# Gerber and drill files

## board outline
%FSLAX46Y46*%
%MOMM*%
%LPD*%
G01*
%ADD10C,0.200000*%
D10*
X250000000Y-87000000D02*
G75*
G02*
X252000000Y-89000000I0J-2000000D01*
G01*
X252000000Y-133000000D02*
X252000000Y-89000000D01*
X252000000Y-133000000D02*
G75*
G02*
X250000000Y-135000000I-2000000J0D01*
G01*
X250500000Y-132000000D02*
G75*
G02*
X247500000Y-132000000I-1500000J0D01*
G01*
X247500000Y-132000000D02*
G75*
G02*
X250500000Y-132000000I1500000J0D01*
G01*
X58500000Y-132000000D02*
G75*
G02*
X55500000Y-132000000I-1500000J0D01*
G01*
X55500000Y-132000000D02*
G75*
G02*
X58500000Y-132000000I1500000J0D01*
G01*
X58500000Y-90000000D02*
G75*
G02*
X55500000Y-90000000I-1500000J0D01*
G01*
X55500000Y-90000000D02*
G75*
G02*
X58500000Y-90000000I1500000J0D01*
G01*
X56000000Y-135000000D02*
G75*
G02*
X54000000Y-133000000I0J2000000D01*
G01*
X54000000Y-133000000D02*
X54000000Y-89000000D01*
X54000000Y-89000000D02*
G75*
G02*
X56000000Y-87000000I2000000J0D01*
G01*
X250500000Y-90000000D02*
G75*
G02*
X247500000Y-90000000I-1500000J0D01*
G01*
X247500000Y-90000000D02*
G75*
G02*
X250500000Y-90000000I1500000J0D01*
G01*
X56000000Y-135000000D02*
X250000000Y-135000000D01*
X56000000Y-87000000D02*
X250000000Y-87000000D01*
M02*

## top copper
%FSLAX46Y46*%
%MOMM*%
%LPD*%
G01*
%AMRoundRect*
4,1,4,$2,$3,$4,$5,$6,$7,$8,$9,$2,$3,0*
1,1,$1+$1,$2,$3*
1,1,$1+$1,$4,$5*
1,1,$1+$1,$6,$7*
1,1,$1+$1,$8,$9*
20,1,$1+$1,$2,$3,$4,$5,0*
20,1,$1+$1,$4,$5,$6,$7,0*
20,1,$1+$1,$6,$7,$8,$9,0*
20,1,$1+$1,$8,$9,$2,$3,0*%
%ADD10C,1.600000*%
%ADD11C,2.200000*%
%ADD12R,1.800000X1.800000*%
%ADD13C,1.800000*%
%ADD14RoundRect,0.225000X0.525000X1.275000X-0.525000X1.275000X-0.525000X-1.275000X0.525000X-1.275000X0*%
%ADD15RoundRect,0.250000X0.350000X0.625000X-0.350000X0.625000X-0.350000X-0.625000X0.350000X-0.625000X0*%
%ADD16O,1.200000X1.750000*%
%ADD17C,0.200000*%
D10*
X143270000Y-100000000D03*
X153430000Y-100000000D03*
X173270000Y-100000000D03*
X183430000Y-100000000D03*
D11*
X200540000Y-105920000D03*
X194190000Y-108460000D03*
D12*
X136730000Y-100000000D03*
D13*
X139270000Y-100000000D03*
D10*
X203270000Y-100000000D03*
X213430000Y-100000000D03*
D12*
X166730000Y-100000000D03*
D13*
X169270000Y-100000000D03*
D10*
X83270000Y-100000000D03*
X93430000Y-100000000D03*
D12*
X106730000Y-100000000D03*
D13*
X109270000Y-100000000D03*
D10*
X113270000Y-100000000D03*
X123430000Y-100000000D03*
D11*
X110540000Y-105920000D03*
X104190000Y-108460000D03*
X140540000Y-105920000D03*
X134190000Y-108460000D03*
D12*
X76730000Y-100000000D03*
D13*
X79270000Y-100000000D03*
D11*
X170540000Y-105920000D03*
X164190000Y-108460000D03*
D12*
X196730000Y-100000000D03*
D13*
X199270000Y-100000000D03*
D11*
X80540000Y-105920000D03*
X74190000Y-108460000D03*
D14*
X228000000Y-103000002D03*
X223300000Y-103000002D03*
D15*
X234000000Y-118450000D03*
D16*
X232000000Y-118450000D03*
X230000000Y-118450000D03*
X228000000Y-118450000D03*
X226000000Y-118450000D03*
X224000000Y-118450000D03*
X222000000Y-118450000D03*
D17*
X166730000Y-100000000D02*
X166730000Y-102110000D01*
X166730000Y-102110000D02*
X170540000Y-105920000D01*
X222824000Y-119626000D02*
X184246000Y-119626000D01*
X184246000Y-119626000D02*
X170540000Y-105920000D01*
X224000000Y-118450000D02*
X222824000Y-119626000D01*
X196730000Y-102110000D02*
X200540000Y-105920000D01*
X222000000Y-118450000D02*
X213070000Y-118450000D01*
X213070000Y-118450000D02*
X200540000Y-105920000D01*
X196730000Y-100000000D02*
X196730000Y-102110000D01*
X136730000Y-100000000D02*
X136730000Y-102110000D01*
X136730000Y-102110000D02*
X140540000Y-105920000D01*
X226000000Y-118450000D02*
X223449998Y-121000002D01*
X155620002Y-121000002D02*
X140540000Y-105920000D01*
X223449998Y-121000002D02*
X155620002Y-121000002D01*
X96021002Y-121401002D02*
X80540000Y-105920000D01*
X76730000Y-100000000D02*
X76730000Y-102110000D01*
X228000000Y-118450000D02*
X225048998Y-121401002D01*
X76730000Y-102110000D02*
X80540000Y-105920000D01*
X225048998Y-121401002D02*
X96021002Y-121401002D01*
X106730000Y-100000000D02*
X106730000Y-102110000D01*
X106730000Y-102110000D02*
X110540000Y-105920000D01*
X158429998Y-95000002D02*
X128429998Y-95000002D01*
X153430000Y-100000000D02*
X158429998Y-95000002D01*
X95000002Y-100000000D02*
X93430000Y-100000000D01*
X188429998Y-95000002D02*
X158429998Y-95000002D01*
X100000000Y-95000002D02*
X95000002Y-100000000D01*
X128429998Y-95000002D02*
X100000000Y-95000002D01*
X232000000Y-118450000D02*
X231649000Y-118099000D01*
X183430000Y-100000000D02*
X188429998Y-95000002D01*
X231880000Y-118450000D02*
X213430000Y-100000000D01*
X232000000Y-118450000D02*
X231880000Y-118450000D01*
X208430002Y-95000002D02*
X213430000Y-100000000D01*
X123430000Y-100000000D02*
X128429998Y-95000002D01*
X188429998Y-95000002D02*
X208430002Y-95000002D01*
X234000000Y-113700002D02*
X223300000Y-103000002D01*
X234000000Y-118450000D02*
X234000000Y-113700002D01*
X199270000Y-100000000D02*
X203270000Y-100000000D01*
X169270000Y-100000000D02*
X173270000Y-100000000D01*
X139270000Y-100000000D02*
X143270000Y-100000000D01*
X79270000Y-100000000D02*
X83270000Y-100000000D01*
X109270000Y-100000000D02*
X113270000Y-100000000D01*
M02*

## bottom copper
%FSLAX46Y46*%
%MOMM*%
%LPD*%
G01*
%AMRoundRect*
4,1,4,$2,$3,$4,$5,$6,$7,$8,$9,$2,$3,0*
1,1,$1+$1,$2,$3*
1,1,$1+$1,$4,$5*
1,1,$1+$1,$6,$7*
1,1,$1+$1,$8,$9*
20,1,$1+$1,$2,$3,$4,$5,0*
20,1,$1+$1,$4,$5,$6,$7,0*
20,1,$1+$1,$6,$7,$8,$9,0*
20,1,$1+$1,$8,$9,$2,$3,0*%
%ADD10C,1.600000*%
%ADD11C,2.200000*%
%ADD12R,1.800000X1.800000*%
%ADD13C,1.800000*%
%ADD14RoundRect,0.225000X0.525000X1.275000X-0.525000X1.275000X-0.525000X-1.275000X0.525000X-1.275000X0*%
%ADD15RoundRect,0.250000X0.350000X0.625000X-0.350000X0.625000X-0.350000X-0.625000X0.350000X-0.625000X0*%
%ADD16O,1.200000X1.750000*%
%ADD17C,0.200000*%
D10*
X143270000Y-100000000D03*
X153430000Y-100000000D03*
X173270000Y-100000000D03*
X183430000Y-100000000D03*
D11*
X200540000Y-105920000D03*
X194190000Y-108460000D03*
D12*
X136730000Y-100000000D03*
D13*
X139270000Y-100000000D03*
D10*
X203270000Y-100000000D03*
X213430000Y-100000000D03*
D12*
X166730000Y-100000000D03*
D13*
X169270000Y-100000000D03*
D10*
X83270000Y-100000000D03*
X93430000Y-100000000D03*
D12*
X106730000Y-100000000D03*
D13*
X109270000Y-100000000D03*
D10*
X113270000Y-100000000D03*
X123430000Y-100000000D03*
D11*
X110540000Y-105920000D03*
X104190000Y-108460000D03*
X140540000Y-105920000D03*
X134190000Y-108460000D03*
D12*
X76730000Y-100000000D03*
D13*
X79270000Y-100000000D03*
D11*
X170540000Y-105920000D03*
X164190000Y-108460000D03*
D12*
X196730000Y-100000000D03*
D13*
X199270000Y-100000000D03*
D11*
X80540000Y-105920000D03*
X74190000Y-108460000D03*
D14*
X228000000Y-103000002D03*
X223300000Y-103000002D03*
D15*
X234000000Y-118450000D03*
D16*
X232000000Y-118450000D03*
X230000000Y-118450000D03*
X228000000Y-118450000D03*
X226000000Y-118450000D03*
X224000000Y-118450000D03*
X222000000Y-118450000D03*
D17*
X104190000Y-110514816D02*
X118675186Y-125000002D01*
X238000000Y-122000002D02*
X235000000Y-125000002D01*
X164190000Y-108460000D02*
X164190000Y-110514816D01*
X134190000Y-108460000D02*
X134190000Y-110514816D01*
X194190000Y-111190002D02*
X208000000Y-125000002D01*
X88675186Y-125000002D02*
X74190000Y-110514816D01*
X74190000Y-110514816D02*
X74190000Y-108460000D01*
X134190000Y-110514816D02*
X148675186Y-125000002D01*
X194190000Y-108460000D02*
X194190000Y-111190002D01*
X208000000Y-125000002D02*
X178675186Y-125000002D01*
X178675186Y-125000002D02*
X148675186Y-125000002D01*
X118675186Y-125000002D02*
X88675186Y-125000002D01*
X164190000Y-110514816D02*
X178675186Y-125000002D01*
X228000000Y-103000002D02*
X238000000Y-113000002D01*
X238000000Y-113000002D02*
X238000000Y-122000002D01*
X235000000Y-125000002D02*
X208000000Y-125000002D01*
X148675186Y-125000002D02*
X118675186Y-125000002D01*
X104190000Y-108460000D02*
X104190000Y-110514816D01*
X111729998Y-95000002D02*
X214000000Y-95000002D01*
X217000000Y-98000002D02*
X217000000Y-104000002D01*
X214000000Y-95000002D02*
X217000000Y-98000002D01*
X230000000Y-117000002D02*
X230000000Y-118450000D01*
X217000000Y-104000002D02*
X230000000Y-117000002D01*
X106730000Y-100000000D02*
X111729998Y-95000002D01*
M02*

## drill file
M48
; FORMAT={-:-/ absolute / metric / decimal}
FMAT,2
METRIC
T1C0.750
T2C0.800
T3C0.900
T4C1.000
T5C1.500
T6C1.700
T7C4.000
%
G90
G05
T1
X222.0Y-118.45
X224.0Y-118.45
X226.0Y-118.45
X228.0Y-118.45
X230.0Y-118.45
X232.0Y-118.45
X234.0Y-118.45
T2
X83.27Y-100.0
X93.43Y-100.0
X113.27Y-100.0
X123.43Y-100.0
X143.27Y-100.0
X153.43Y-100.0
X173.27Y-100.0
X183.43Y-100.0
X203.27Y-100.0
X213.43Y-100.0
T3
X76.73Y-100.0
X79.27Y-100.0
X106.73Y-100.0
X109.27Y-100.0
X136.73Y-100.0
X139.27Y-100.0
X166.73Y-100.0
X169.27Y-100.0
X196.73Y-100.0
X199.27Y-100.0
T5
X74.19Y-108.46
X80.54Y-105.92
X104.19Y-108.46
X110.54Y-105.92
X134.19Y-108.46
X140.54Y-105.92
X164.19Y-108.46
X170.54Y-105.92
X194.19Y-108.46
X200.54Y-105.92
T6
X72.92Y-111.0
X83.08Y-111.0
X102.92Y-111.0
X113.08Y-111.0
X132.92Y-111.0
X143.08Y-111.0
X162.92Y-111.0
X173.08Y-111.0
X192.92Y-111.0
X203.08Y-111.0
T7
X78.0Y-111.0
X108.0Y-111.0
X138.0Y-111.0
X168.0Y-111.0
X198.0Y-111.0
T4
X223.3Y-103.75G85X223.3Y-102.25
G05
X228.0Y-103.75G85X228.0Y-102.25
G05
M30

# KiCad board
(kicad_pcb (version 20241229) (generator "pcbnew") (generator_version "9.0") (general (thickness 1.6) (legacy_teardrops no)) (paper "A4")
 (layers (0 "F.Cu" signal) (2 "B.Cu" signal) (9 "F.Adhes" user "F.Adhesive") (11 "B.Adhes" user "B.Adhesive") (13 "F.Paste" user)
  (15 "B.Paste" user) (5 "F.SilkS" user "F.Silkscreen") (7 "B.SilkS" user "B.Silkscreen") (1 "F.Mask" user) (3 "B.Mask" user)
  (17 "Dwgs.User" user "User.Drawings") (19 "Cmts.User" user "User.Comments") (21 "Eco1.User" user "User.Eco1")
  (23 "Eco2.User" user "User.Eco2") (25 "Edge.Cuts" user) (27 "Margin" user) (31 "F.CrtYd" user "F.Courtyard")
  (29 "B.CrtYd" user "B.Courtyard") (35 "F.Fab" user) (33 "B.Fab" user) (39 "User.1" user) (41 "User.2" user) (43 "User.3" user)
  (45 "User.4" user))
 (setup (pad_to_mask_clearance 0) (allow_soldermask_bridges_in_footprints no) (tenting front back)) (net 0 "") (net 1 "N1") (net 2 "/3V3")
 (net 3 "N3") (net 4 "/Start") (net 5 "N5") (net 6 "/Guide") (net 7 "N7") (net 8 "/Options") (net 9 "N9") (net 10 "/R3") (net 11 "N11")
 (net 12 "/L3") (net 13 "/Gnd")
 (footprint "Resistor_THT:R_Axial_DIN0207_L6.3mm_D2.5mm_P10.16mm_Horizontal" (layer "F.Cu") (at 143.27 100)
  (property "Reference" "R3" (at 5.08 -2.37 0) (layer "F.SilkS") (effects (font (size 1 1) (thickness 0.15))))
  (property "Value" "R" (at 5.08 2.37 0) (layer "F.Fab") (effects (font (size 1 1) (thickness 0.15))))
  (pad "1" thru_hole circle (at 0 0) (size 1.6 1.6) (drill 0.8) (layers "*.Cu" "*.Mask") (remove_unused_layers no) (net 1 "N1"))
  (pad "2" thru_hole circle (at 10.16 0) (size 1.6 1.6) (drill 0.8) (layers "*.Cu" "*.Mask") (remove_unused_layers no) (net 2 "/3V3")))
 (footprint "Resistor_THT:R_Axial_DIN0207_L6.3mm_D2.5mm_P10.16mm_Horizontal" (layer "F.Cu") (at 173.27 100)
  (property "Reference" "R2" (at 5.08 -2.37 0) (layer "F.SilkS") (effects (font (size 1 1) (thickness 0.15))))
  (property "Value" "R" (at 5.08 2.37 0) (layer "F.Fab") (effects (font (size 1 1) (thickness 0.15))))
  (pad "1" thru_hole circle (at 0 0) (size 1.6 1.6) (drill 0.8) (layers "*.Cu" "*.Mask") (remove_unused_layers no) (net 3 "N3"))
  (pad "2" thru_hole circle (at 10.16 0) (size 1.6 1.6) (drill 0.8) (layers "*.Cu" "*.Mask") (remove_unused_layers no) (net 2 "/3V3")))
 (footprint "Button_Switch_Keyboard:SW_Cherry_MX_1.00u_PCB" (layer "F.Cu") (at 200.54 105.92)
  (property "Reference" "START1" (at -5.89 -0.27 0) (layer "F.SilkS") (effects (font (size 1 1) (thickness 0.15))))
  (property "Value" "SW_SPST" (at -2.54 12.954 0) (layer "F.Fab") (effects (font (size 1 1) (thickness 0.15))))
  (pad "" np_thru_hole circle (at -7.62 5.08) (size 1.7 1.7) (drill 1.7) (layers "*.Cu" "*.Mask"))
  (pad "" np_thru_hole circle (at -2.54 5.08) (size 4 4) (drill 4) (layers "*.Cu" "*.Mask"))
  (pad "" np_thru_hole circle (at 2.54 5.08) (size 1.7 1.7) (drill 1.7) (layers "*.Cu" "*.Mask"))
  (pad "1" thru_hole circle (at 0 0) (size 2.2 2.2) (drill 1.5) (layers "*.Cu" "*.Mask") (remove_unused_layers no) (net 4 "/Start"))
  (pad "2" thru_hole circle (at -6.35 2.54) (size 2.2 2.2) (drill 1.5) (layers "*.Cu" "*.Mask") (remove_unused_layers no) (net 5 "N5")))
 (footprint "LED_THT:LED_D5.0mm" (layer "F.Cu") (at 136.73 100)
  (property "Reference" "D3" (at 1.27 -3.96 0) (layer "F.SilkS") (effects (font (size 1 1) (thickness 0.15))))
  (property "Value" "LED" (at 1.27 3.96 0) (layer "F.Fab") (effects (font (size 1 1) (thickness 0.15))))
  (pad "1" thru_hole rect (at 0 0) (size 1.8 1.8) (drill 0.9) (layers "*.Cu" "*.Mask") (remove_unused_layers no) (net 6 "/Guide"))
  (pad "2" thru_hole circle (at 2.54 0) (size 1.8 1.8) (drill 0.9) (layers "*.Cu" "*.Mask") (remove_unused_layers no) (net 1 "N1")))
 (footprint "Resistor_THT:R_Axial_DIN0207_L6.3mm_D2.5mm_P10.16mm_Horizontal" (layer "F.Cu") (at 203.27 100)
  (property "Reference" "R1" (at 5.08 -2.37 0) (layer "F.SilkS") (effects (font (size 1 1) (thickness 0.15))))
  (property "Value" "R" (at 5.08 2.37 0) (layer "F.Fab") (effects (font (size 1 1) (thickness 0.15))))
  (pad "1" thru_hole circle (at 0 0) (size 1.6 1.6) (drill 0.8) (layers "*.Cu" "*.Mask") (remove_unused_layers no) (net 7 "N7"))
  (pad "2" thru_hole circle (at 10.16 0) (size 1.6 1.6) (drill 0.8) (layers "*.Cu" "*.Mask") (remove_unused_layers no) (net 2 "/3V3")))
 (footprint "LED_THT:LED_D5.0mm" (layer "F.Cu") (at 166.73 100)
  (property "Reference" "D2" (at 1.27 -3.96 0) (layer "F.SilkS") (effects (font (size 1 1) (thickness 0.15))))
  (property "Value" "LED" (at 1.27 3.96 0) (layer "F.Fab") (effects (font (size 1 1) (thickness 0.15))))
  (pad "1" thru_hole rect (at 0 0) (size 1.8 1.8) (drill 0.9) (layers "*.Cu" "*.Mask") (remove_unused_layers no) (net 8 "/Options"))
  (pad "2" thru_hole circle (at 2.54 0) (size 1.8 1.8) (drill 0.9) (layers "*.Cu" "*.Mask") (remove_unused_layers no) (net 3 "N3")))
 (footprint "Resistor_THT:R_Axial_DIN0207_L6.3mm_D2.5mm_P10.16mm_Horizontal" (layer "F.Cu") (at 83.27 100)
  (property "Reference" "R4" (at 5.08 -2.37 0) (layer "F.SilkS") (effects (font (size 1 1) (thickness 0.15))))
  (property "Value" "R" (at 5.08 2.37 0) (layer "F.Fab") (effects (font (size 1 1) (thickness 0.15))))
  (pad "1" thru_hole circle (at 0 0) (size 1.6 1.6) (drill 0.8) (layers "*.Cu" "*.Mask") (remove_unused_layers no) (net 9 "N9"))
  (pad "2" thru_hole circle (at 10.16 0) (size 1.6 1.6) (drill 0.8) (layers "*.Cu" "*.Mask") (remove_unused_layers no) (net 2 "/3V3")))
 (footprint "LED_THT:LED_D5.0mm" (layer "F.Cu") (at 106.73 100)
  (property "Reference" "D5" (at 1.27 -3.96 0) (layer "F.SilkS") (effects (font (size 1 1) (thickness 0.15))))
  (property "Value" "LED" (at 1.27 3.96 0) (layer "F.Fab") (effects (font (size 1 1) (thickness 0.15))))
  (pad "1" thru_hole rect (at 0 0) (size 1.8 1.8) (drill 0.9) (layers "*.Cu" "*.Mask") (remove_unused_layers no) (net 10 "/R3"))
  (pad "2" thru_hole circle (at 2.54 0) (size 1.8 1.8) (drill 0.9) (layers "*.Cu" "*.Mask") (remove_unused_layers no) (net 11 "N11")))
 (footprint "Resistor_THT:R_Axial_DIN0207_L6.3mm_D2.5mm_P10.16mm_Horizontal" (layer "F.Cu") (at 113.27 100)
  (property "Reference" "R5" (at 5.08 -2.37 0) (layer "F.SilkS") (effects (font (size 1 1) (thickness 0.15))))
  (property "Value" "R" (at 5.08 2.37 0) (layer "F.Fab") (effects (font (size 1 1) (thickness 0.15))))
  (pad "1" thru_hole circle (at 0 0) (size 1.6 1.6) (drill 0.8) (layers "*.Cu" "*.Mask") (remove_unused_layers no) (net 11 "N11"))
  (pad "2" thru_hole circle (at 10.16 0) (size 1.6 1.6) (drill 0.8) (layers "*.Cu" "*.Mask") (remove_unused_layers no) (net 2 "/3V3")))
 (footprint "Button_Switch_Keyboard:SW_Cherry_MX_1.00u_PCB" (layer "F.Cu") (at 110.54 105.92)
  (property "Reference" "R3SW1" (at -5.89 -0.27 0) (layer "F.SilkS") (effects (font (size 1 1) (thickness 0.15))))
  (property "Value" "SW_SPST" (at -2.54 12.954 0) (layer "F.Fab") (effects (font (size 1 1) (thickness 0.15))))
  (pad "" np_thru_hole circle (at -7.62 5.08) (size 1.7 1.7) (drill 1.7) (layers "*.Cu" "*.Mask"))
  (pad "" np_thru_hole circle (at -2.54 5.08) (size 4 4) (drill 4) (layers "*.Cu" "*.Mask"))
  (pad "" np_thru_hole circle (at 2.54 5.08) (size 1.7 1.7) (drill 1.7) (layers "*.Cu" "*.Mask"))
  (pad "1" thru_hole circle (at 0 0) (size 2.2 2.2) (drill 1.5) (layers "*.Cu" "*.Mask") (remove_unused_layers no) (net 10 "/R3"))
  (pad "2" thru_hole circle (at -6.35 2.54) (size 2.2 2.2) (drill 1.5) (layers "*.Cu" "*.Mask") (remove_unused_layers no) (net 5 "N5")))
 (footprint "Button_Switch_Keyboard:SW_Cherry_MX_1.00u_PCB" (layer "F.Cu") (at 140.54 105.92)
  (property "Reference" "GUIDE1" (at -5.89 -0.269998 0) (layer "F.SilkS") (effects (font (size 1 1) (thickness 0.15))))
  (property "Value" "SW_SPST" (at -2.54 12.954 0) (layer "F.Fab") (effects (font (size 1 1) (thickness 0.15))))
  (pad "" np_thru_hole circle (at -7.62 5.08) (size 1.7 1.7) (drill 1.7) (layers "*.Cu" "*.Mask"))
  (pad "" np_thru_hole circle (at -2.54 5.08) (size 4 4) (drill 4) (layers "*.Cu" "*.Mask"))
  (pad "" np_thru_hole circle (at 2.54 5.08) (size 1.7 1.7) (drill 1.7) (layers "*.Cu" "*.Mask"))
  (pad "1" thru_hole circle (at 0 0) (size 2.2 2.2) (drill 1.5) (layers "*.Cu" "*.Mask") (remove_unused_layers no) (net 6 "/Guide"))
  (pad "2" thru_hole circle (at -6.35 2.54) (size 2.2 2.2) (drill 1.5) (layers "*.Cu" "*.Mask") (remove_unused_layers no) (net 5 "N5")))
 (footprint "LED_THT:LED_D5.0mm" (layer "F.Cu") (at 76.73 100)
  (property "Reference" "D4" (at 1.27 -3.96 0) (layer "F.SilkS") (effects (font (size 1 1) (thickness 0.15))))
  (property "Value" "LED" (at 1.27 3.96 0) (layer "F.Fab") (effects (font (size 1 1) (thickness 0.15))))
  (pad "1" thru_hole rect (at 0 0) (size 1.8 1.8) (drill 0.9) (layers "*.Cu" "*.Mask") (remove_unused_layers no) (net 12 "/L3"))
  (pad "2" thru_hole circle (at 2.54 0) (size 1.8 1.8) (drill 0.9) (layers "*.Cu" "*.Mask") (remove_unused_layers no) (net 9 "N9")))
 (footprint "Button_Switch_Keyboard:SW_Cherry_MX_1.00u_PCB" (layer "F.Cu") (at 170.54 105.92)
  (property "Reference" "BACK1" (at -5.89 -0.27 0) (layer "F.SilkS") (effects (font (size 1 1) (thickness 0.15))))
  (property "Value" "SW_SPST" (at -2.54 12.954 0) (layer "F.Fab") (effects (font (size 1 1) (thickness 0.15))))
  (pad "" np_thru_hole circle (at -7.62 5.08) (size 1.7 1.7) (drill 1.7) (layers "*.Cu" "*.Mask"))
  (pad "" np_thru_hole circle (at -2.54 5.08) (size 4 4) (drill 4) (layers "*.Cu" "*.Mask"))
  (pad "" np_thru_hole circle (at 2.54 5.08) (size 1.7 1.7) (drill 1.7) (layers "*.Cu" "*.Mask"))
  (pad "1" thru_hole circle (at 0 0) (size 2.2 2.2) (drill 1.5) (layers "*.Cu" "*.Mask") (remove_unused_layers no) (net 8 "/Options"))
  (pad "2" thru_hole circle (at -6.35 2.54) (size 2.2 2.2) (drill 1.5) (layers "*.Cu" "*.Mask") (remove_unused_layers no) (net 5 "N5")))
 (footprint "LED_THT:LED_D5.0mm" (layer "F.Cu") (at 196.73 100)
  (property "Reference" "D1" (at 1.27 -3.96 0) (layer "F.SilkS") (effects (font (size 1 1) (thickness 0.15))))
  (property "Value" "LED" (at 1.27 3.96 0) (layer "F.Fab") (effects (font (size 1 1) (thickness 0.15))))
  (pad "1" thru_hole rect (at 0 0) (size 1.8 1.8) (drill 0.9) (layers "*.Cu" "*.Mask") (remove_unused_layers no) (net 4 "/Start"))
  (pad "2" thru_hole circle (at 2.54 0) (size 1.8 1.8) (drill 0.9) (layers "*.Cu" "*.Mask") (remove_unused_layers no) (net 7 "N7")))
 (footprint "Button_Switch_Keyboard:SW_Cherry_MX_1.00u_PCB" (layer "F.Cu") (at 80.54 105.92)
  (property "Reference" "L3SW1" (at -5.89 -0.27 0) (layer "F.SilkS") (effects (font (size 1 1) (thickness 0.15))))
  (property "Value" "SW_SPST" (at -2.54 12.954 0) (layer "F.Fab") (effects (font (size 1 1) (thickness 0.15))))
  (pad "" np_thru_hole circle (at -7.62 5.08) (size 1.7 1.7) (drill 1.7) (layers "*.Cu" "*.Mask"))
  (pad "" np_thru_hole circle (at -2.54 5.08) (size 4 4) (drill 4) (layers "*.Cu" "*.Mask"))
  (pad "" np_thru_hole circle (at 2.54 5.08) (size 1.7 1.7) (drill 1.7) (layers "*.Cu" "*.Mask"))
  (pad "1" thru_hole circle (at 0 0) (size 2.2 2.2) (drill 1.5) (layers "*.Cu" "*.Mask") (remove_unused_layers no) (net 12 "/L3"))
  (pad "2" thru_hole circle (at -6.35 2.54) (size 2.2 2.2) (drill 1.5) (layers "*.Cu" "*.Mask") (remove_unused_layers no) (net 5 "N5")))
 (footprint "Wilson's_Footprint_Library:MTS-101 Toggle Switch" (layer "F.Cu") (at 234.5 99.000002 180)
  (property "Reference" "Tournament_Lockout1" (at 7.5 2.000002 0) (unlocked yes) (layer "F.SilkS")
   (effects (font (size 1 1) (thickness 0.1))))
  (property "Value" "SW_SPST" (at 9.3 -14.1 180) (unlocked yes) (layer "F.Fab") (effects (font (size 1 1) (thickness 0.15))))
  (pad "1" thru_hole roundrect (at 6.5 -4 180) (size 1.5 3) (drill oval 1 2.5) (layers "*.Cu" "*.Mask") (remove_unused_layers no)
   (roundrect_rratio 0.15) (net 5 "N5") (thermal_bridge_angle 45))
  (pad "2" thru_hole roundrect (at 11.2 -4 180) (size 1.5 3) (drill oval 1 2.5) (layers "*.Cu" "*.Mask") (remove_unused_layers no)
   (roundrect_rratio 0.15) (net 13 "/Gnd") (thermal_bridge_angle 45)))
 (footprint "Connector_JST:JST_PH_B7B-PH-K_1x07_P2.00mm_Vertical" (layer "B.Cu") (at 234 118.45 180)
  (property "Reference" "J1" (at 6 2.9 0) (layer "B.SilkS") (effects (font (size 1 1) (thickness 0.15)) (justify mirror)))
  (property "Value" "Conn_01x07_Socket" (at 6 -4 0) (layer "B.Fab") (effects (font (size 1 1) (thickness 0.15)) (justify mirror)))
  (pad "1" thru_hole roundrect (at 0 0 180) (size 1.2 1.75) (drill 0.75) (layers "*.Cu" "*.Mask") (remove_unused_layers no)
   (roundrect_rratio 0.208333) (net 13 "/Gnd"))
  (pad "2" thru_hole oval (at 2 0 180) (size 1.2 1.75) (drill 0.75) (layers "*.Cu" "*.Mask") (remove_unused_layers no) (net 2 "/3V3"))
  (pad "3" thru_hole oval (at 4 0 180) (size 1.2 1.75) (drill 0.75) (layers "*.Cu" "*.Mask") (remove_unused_layers no) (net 10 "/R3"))
  (pad "4" thru_hole oval (at 6 0 180) (size 1.2 1.75) (drill 0.75) (layers "*.Cu" "*.Mask") (remove_unused_layers no) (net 12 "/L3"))
  (pad "5" thru_hole oval (at 8 0 180) (size 1.2 1.75) (drill 0.75) (layers "*.Cu" "*.Mask") (remove_unused_layers no) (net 6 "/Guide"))
  (pad "6" thru_hole oval (at 10 0 180) (size 1.2 1.75) (drill 0.75) (layers "*.Cu" "*.Mask") (remove_unused_layers no) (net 8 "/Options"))
  (pad "7" thru_hole oval (at 12 0 180) (size 1.2 1.75) (drill 0.75) (layers "*.Cu" "*.Mask") (remove_unused_layers no) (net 4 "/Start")))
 (gr_arc (start 250 87) (mid 251.414214 87.585786) (end 252 89) (stroke (width 0.2) (type default)) (layer "Edge.Cuts"))
 (gr_line (start 252 133) (end 252 89) (stroke (width 0.2) (type default)) (layer "Edge.Cuts"))
 (gr_arc (start 252 133) (mid 251.414214 134.414214) (end 250 135) (stroke (width 0.2) (type default)) (layer "Edge.Cuts"))
 (gr_circle (center 249 132) (end 250.5 132) (stroke (width 0.2) (type default)) (fill no) (layer "Edge.Cuts"))
 (gr_circle (center 57 132) (end 58.5 132) (stroke (width 0.2) (type default)) (fill no) (layer "Edge.Cuts"))
 (gr_circle (center 57 90) (end 58.5 90) (stroke (width 0.2) (type default)) (fill no) (layer "Edge.Cuts"))
 (gr_arc (start 56 135) (mid 54.585786 134.414214) (end 54 133) (stroke (width 0.2) (type default)) (layer "Edge.Cuts"))
 (gr_line (start 54 133) (end 54 89) (stroke (width 0.2) (type default)) (layer "Edge.Cuts"))
 (gr_arc (start 54 89) (mid 54.585786 87.585786) (end 56 87) (stroke (width 0.2) (type default)) (layer "Edge.Cuts"))
 (gr_circle (center 249 90) (end 250.5 90) (stroke (width 0.2) (type default)) (fill no) (layer "Edge.Cuts"))
 (gr_line (start 56 135) (end 250 135) (stroke (width 0.2) (type default)) (layer "Edge.Cuts"))
 (gr_line (start 56 87) (end 250 87) (stroke (width 0.2) (type default)) (layer "Edge.Cuts"))
 (segment (start 166.73 100) (end 166.73 102.11) (width 0.2) (layer "F.Cu") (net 8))
 (segment (start 166.73 102.11) (end 170.54 105.92) (width 0.2) (layer "F.Cu") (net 8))
 (segment (start 222.824 119.626) (end 184.246 119.626) (width 0.2) (layer "F.Cu") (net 8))
 (segment (start 184.246 119.626) (end 170.54 105.92) (width 0.2) (layer "F.Cu") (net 8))
 (segment (start 224 118.45) (end 222.824 119.626) (width 0.2) (layer "F.Cu") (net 8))
 (segment (start 104.19 110.514816) (end 118.675186 125.000002) (width 0.2) (layer "B.Cu") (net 5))
 (segment (start 238 122.000002) (end 235 125.000002) (width 0.2) (layer "B.Cu") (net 5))
 (segment (start 164.19 108.46) (end 164.19 110.514816) (width 0.2) (layer "B.Cu") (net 5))
 (segment (start 134.19 108.46) (end 134.19 110.514816) (width 0.2) (layer "B.Cu") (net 5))
 (segment (start 194.19 111.190002) (end 208 125.000002) (width 0.2) (layer "B.Cu") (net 5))
 (segment (start 88.675186 125.000002) (end 74.19 110.514816) (width 0.2) (layer "B.Cu") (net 5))
 (segment (start 74.19 110.514816) (end 74.19 108.46) (width 0.2) (layer "B.Cu") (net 5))
 (segment (start 134.19 110.514816) (end 148.675186 125.000002) (width 0.2) (layer "B.Cu") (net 5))
 (segment (start 194.19 108.46) (end 194.19 111.190002) (width 0.2) (layer "B.Cu") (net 5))
 (segment (start 208 125.000002) (end 178.675186 125.000002) (width 0.2) (layer "B.Cu") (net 5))
 (segment (start 178.675186 125.000002) (end 148.675186 125.000002) (width 0.2) (layer "B.Cu") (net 5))
 (segment (start 118.675186 125.000002) (end 88.675186 125.000002) (width 0.2) (layer "B.Cu") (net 5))
 (segment (start 164.19 110.514816) (end 178.675186 125.000002) (width 0.2) (layer "B.Cu") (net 5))
 (segment (start 228 103.000002) (end 238 113.000002) (width 0.2) (layer "B.Cu") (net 5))
 (segment (start 238 113.000002) (end 238 122.000002) (width 0.2) (layer "B.Cu") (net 5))
 (segment (start 235 125.000002) (end 208 125.000002) (width 0.2) (layer "B.Cu") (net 5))
 (segment (start 148.675186 125.000002) (end 118.675186 125.000002) (width 0.2) (layer "B.Cu") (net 5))
 (segment (start 104.19 108.46) (end 104.19 110.514816) (width 0.2) (layer "B.Cu") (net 5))
 (segment (start 196.73 102.11) (end 200.54 105.92) (width 0.2) (layer "F.Cu") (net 4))
 (segment (start 222 118.45) (end 213.07 118.45) (width 0.2) (layer "F.Cu") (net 4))
 (segment (start 213.07 118.45) (end 200.54 105.92) (width 0.2) (layer "F.Cu") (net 4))
 (segment (start 196.73 100) (end 196.73 102.11) (width 0.2) (layer "F.Cu") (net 4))
 (segment (start 136.73 100) (end 136.73 102.11) (width 0.2) (layer "F.Cu") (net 6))
 (segment (start 136.73 102.11) (end 140.54 105.92) (width 0.2) (layer "F.Cu") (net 6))
 (segment (start 226 118.45) (end 223.449998 121.000002) (width 0.2) (layer "F.Cu") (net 6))
 (segment (start 155.620002 121.000002) (end 140.54 105.92) (width 0.2) (layer "F.Cu") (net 6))
 (segment (start 223.449998 121.000002) (end 155.620002 121.000002) (width 0.2) (layer "F.Cu") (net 6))
 (segment (start 96.021002 121.401002) (end 80.54 105.92) (width 0.2) (layer "F.Cu") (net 12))
 (segment (start 76.73 100) (end 76.73 102.11) (width 0.2) (layer "F.Cu") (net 12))
 (segment (start 228 118.45) (end 225.048998 121.401002) (width 0.2) (layer "F.Cu") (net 12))
 (segment (start 76.73 102.11) (end 80.54 105.92) (width 0.2) (layer "F.Cu") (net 12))
 (segment (start 225.048998 121.401002) (end 96.021002 121.401002) (width 0.2) (layer "F.Cu") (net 12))
 (segment (start 106.73 100) (end 106.73 102.11) (width 0.2) (layer "F.Cu") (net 10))
 (segment (start 106.73 102.11) (end 110.54 105.92) (width 0.2) (layer "F.Cu") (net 10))
 (segment (start 111.729998 95.000002) (end 214 95.000002) (width 0.2) (layer "B.Cu") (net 10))
 (segment (start 217 98.000002) (end 217 104.000002) (width 0.2) (layer "B.Cu") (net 10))
 (segment (start 214 95.000002) (end 217 98.000002) (width 0.2) (layer "B.Cu") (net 10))
 (segment (start 230 117.000002) (end 230 118.45) (width 0.2) (layer "B.Cu") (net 10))
 (segment (start 217 104.000002) (end 230 117.000002) (width 0.2) (layer "B.Cu") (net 10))
 (segment (start 106.73 100) (end 111.729998 95.000002) (width 0.2) (layer "B.Cu") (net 10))
 (segment (start 158.429998 95.000002) (end 128.429998 95.000002) (width 0.2) (layer "F.Cu") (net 2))
 (segment (start 153.43 100) (end 158.429998 95.000002) (width 0.2) (layer "F.Cu") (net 2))
 (segment (start 95.000002 100) (end 93.43 100) (width 0.2) (layer "F.Cu") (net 2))
 (segment (start 188.429998 95.000002) (end 158.429998 95.000002) (width 0.2) (layer "F.Cu") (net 2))
 (segment (start 100 95.000002) (end 95.000002 100) (width 0.2) (layer "F.Cu") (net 2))
 (segment (start 128.429998 95.000002) (end 100 95.000002) (width 0.2) (layer "F.Cu") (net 2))
 (segment (start 232 118.45) (end 231.649 118.099) (width 0.2) (layer "F.Cu") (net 2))
 (segment (start 183.43 100) (end 188.429998 95.000002) (width 0.2) (layer "F.Cu") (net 2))
 (segment (start 231.88 118.45) (end 213.43 100) (width 0.2) (layer "F.Cu") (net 2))
 (segment (start 232 118.45) (end 231.88 118.45) (width 0.2) (layer "F.Cu") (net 2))
 (segment (start 208.430002 95.000002) (end 213.43 100) (width 0.2) (layer "F.Cu") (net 2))
 (segment (start 123.43 100) (end 128.429998 95.000002) (width 0.2) (layer "F.Cu") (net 2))
 (segment (start 188.429998 95.000002) (end 208.430002 95.000002) (width 0.2) (layer "F.Cu") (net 2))
 (segment (start 234 113.700002) (end 223.3 103.000002) (width 0.2) (layer "F.Cu") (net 13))
 (segment (start 234 118.45) (end 234 113.700002) (width 0.2) (layer "F.Cu") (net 13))
 (segment (start 199.27 100) (end 203.27 100) (width 0.2) (layer "F.Cu") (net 7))
 (segment (start 169.27 100) (end 173.27 100) (width 0.2) (layer "F.Cu") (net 3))
 (segment (start 139.27 100) (end 143.27 100) (width 0.2) (layer "F.Cu") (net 1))
 (segment (start 79.27 100) (end 83.27 100) (width 0.2) (layer "F.Cu") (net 9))
 (segment (start 109.27 100) (end 113.27 100) (width 0.2) (layer "F.Cu") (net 11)))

